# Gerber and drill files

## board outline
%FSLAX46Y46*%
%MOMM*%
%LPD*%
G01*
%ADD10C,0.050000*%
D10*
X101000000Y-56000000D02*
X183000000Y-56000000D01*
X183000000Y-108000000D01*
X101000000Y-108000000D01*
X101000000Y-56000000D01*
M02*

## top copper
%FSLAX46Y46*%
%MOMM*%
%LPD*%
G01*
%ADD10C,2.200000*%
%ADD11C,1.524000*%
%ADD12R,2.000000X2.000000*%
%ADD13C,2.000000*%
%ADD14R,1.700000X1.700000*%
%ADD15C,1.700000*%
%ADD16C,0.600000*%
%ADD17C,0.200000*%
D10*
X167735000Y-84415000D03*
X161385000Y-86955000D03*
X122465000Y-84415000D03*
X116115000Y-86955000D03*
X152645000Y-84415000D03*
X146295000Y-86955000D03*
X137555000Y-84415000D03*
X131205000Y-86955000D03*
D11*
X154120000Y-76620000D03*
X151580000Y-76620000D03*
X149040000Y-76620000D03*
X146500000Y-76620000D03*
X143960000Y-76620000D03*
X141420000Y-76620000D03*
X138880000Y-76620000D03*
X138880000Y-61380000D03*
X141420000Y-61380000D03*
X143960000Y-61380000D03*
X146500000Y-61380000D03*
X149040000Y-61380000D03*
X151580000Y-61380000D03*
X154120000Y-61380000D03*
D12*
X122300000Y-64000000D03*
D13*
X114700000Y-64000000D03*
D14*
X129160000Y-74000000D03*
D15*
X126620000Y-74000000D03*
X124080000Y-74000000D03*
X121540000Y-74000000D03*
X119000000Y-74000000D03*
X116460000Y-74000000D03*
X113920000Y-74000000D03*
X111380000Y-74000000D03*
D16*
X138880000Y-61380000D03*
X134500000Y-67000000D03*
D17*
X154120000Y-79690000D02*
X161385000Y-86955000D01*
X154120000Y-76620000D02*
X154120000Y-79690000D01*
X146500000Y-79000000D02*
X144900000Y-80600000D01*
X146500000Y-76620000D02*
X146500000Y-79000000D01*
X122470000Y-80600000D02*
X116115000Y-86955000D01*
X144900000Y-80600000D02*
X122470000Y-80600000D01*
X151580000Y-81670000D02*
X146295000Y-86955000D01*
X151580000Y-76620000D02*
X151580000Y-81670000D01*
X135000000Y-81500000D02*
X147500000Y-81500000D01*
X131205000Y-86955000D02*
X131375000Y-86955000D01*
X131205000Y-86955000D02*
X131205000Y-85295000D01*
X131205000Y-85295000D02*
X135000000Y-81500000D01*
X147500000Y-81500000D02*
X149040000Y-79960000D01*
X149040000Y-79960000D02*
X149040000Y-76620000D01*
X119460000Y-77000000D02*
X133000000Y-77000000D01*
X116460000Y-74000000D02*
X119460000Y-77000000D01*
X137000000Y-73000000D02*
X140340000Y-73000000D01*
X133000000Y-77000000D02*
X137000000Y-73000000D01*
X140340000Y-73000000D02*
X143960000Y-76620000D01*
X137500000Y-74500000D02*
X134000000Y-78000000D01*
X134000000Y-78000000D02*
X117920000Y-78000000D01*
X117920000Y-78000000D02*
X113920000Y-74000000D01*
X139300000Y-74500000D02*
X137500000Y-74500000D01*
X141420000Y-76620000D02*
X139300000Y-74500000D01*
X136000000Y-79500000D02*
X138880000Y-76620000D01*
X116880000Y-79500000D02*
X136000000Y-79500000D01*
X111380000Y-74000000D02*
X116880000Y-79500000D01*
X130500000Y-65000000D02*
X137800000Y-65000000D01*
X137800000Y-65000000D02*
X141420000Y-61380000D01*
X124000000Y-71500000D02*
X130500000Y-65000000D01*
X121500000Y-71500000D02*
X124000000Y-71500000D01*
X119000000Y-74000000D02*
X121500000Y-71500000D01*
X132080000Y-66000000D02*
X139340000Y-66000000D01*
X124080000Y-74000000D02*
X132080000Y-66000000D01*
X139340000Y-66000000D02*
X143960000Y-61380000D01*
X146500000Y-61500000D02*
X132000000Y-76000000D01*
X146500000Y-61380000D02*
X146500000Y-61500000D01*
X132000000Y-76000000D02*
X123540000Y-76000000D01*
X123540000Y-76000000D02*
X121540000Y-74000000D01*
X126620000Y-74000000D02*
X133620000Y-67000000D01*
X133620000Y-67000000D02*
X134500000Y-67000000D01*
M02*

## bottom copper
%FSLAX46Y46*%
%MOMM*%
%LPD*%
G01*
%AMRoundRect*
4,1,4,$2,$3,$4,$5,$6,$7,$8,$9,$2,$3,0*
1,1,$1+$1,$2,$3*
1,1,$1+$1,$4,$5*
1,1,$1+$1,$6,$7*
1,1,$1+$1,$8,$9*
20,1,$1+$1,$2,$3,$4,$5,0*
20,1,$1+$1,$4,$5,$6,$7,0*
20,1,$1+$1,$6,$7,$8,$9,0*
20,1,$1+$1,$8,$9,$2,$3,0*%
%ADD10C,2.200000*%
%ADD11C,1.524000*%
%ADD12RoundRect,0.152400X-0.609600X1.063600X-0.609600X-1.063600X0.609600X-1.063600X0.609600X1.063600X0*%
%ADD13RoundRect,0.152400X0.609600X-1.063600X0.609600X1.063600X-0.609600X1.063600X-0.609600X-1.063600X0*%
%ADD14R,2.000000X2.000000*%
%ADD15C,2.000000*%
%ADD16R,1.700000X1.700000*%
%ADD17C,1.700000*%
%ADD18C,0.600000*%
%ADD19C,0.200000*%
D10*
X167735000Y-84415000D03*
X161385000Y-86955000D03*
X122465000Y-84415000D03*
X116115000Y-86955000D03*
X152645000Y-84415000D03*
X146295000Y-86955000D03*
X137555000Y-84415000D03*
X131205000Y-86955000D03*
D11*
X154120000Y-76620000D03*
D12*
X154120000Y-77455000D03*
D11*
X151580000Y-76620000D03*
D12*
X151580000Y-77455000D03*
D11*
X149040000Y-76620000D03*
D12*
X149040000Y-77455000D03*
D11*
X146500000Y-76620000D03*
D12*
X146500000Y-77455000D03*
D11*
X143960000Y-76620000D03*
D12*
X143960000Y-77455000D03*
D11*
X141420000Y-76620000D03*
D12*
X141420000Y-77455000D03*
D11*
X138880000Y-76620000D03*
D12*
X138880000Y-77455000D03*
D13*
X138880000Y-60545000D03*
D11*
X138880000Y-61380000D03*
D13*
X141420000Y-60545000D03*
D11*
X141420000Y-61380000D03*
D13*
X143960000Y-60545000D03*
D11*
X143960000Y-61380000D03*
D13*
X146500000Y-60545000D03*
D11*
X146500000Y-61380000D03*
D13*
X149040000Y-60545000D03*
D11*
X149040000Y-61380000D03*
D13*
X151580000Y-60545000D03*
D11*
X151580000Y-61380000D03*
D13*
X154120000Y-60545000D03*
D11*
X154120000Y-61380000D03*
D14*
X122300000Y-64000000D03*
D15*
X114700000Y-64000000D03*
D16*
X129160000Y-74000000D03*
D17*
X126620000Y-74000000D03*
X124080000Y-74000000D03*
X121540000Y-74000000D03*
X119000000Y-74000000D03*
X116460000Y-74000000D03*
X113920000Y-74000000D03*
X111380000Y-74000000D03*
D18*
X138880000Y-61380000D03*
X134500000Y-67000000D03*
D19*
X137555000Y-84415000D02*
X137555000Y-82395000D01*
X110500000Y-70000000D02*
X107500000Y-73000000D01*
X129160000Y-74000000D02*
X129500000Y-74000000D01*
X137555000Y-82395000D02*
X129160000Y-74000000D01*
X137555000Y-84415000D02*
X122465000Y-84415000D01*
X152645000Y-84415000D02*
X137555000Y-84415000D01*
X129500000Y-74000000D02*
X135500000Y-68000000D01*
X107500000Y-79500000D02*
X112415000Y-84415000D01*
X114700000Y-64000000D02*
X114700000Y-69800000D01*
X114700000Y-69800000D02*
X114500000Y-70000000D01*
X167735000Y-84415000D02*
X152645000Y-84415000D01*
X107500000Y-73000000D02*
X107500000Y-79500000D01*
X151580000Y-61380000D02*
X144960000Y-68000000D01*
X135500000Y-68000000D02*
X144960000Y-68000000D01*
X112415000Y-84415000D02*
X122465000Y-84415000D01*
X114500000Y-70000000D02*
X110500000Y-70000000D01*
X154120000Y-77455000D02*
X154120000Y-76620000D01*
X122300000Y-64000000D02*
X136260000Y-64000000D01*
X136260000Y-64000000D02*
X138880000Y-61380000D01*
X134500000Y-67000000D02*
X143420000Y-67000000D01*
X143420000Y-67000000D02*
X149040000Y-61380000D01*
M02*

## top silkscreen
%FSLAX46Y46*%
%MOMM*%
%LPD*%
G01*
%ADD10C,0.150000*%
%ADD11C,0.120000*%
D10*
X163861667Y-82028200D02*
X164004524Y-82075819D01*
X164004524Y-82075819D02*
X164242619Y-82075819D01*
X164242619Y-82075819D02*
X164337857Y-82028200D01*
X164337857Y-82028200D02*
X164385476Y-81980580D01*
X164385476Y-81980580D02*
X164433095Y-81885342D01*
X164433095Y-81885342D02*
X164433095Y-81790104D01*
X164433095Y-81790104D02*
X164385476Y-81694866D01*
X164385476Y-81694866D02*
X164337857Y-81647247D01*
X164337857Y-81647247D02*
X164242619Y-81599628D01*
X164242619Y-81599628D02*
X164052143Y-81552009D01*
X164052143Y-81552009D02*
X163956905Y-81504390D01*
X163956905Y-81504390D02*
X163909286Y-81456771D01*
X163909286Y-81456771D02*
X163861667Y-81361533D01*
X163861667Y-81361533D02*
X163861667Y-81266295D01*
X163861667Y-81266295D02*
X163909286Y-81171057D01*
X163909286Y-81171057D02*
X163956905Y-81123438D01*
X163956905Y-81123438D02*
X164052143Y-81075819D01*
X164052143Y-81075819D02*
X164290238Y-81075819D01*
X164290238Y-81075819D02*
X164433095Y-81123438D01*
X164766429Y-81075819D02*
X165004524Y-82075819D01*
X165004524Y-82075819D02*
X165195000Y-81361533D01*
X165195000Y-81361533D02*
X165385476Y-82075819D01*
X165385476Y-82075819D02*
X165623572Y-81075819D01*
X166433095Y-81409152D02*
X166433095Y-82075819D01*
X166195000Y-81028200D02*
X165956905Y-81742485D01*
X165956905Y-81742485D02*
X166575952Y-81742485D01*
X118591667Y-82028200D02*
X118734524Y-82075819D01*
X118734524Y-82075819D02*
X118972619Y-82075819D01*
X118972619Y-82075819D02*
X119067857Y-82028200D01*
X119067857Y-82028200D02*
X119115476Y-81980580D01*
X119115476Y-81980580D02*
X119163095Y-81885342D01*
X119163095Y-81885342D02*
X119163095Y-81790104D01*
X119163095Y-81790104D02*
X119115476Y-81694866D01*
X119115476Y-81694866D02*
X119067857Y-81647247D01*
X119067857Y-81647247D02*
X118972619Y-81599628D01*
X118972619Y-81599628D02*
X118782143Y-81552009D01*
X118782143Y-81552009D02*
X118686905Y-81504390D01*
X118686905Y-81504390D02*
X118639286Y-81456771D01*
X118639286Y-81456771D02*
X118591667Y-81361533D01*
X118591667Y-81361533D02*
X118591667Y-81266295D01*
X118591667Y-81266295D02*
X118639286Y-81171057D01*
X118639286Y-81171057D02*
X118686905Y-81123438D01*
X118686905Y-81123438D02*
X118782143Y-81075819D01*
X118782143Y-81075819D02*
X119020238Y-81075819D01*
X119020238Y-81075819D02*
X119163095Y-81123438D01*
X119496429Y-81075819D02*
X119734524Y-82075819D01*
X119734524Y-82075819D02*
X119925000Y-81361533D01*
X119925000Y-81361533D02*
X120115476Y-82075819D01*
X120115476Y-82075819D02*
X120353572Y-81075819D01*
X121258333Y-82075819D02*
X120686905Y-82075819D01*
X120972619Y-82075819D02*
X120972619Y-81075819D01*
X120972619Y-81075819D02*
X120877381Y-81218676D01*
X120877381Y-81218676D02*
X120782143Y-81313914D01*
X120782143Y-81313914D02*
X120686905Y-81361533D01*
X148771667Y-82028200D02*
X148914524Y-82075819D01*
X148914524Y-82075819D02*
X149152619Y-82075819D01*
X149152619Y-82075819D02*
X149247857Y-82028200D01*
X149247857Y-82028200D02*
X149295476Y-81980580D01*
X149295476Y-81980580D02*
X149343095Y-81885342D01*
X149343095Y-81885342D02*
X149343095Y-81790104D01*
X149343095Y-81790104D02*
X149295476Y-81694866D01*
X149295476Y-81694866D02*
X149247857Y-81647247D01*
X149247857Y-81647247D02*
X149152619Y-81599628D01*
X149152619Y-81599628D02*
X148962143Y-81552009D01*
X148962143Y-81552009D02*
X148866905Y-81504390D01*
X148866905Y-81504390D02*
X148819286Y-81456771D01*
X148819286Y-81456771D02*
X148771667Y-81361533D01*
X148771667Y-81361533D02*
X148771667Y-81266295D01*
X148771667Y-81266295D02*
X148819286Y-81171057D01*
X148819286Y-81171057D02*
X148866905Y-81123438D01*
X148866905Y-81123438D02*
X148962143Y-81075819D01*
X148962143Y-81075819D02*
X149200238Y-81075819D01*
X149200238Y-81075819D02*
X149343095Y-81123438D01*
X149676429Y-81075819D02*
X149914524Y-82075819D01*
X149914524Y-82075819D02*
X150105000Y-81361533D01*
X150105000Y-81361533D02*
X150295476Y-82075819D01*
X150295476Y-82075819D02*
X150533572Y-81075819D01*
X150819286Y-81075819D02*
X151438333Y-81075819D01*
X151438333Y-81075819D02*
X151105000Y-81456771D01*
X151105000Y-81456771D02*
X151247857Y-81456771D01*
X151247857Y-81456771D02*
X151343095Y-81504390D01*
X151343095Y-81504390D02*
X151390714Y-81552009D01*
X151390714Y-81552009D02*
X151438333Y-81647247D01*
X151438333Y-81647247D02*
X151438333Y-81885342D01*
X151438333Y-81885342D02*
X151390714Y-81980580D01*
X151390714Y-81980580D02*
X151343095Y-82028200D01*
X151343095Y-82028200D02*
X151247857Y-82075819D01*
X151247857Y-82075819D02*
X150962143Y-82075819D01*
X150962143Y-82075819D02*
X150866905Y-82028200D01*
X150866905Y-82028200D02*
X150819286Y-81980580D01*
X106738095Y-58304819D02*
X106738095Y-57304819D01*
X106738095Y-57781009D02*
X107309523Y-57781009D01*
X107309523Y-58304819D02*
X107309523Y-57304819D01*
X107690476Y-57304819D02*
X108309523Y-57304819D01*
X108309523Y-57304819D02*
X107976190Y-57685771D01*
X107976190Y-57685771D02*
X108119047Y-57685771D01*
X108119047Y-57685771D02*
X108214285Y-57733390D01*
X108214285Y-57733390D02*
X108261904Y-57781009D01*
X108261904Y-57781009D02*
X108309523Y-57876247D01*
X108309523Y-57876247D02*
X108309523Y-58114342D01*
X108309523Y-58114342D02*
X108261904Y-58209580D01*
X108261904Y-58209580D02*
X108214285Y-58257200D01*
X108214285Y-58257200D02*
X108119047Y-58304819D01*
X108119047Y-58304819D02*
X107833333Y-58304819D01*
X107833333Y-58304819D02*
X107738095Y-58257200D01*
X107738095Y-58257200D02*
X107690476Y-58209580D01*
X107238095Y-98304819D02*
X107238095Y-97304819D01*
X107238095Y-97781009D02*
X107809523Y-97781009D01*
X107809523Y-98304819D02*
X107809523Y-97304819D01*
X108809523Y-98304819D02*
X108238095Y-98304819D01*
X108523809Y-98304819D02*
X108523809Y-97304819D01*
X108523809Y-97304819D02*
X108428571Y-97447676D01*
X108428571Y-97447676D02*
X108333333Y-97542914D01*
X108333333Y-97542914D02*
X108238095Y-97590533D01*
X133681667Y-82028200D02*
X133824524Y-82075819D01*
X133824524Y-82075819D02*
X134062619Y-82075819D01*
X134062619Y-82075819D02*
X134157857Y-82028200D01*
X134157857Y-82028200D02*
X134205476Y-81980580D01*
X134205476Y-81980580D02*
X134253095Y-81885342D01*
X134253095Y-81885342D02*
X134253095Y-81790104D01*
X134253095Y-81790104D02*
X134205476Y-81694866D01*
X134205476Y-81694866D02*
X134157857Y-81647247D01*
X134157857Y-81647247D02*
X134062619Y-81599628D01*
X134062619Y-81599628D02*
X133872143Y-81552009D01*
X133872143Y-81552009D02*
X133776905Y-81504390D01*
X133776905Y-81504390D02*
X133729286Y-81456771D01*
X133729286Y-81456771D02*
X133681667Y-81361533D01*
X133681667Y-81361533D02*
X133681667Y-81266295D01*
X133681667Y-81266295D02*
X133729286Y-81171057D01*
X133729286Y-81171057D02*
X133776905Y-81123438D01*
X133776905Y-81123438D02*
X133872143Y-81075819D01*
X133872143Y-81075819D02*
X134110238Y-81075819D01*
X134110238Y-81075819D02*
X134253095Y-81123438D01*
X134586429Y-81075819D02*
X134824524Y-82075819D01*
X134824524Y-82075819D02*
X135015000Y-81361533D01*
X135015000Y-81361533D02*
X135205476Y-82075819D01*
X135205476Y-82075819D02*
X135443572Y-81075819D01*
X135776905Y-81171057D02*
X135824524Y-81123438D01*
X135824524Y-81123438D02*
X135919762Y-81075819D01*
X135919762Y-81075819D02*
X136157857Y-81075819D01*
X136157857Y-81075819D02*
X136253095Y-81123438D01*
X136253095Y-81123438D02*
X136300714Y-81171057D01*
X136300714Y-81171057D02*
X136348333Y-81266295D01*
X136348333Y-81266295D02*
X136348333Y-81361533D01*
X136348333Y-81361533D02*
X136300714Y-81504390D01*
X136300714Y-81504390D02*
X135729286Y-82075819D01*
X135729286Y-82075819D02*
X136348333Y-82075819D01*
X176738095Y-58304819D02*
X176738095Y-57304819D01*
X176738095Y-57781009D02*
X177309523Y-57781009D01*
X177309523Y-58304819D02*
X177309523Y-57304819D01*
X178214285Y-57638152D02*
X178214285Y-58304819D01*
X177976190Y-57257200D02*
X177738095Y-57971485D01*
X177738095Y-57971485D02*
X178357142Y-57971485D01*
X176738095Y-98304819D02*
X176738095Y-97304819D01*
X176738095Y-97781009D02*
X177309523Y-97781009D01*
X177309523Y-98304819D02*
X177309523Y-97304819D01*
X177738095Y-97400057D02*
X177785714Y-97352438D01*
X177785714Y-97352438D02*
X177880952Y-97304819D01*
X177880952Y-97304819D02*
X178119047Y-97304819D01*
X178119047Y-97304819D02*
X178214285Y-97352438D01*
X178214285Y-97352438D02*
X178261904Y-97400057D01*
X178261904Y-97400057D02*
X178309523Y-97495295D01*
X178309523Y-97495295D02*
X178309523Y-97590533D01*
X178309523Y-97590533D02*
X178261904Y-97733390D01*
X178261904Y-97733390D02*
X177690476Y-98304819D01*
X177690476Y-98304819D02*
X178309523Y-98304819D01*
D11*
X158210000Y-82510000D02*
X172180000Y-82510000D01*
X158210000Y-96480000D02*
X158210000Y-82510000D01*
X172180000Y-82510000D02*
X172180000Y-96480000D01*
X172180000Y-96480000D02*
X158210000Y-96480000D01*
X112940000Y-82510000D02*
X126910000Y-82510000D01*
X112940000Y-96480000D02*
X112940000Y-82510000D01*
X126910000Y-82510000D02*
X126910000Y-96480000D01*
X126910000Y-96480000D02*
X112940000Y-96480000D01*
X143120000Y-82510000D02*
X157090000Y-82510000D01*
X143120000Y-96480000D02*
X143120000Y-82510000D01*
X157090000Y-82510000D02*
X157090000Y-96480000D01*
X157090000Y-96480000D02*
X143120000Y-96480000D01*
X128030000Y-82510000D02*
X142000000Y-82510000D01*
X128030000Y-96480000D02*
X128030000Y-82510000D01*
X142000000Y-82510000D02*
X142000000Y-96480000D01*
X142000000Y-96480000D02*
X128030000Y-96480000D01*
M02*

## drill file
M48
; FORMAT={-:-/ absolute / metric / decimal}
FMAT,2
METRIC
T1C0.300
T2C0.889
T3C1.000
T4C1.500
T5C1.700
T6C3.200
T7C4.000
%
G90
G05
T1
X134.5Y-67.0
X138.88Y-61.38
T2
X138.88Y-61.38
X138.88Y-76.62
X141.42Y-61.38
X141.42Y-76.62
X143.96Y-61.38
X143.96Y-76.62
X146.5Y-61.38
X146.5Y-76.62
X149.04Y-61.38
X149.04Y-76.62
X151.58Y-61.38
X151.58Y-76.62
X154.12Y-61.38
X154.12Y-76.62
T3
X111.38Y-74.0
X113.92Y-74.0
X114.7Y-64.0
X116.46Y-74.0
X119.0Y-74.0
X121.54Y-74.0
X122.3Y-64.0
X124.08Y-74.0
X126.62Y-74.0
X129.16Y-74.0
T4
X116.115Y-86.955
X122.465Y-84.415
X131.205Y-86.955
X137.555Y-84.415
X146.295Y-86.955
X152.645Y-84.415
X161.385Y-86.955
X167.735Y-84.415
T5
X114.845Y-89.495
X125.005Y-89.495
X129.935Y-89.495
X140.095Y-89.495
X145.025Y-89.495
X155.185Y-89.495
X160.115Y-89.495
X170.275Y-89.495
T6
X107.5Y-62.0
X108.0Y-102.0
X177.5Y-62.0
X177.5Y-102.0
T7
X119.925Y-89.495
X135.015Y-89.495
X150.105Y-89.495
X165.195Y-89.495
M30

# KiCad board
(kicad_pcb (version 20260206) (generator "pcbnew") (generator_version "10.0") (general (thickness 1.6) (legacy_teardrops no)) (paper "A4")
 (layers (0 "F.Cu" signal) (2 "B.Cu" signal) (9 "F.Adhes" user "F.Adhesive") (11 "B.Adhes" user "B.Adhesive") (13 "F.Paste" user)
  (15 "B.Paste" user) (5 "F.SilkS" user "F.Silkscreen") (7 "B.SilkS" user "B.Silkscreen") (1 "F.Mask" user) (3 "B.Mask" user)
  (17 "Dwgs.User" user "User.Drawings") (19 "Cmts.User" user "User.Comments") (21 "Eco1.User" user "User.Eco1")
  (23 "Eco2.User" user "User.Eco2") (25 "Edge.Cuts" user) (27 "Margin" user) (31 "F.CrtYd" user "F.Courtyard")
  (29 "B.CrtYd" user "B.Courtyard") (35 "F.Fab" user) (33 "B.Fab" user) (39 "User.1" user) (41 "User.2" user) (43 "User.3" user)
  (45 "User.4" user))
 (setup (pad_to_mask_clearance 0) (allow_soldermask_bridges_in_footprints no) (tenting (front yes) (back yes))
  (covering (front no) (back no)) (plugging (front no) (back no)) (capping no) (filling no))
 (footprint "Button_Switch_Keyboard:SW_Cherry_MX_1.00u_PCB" (layer "F.Cu") (at 167.735 84.415)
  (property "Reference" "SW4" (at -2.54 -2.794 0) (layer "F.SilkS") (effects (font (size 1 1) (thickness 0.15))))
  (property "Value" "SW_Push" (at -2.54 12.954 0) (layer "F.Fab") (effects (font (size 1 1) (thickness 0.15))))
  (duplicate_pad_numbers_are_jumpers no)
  (fp_line (start -9.525 -1.905) (end 4.445 -1.905) (stroke (width 0.12) (type solid)) (layer "F.SilkS"))
  (fp_line (start -9.525 12.065) (end -9.525 -1.905) (stroke (width 0.12) (type solid)) (layer "F.SilkS"))
  (fp_line (start 4.445 -1.905) (end 4.445 12.065) (stroke (width 0.12) (type solid)) (layer "F.SilkS"))
  (fp_line (start 4.445 12.065) (end -9.525 12.065) (stroke (width 0.12) (type solid)) (layer "F.SilkS"))
  (pad "" np_thru_hole circle (at -7.62 5.08) (size 1.7 1.7) (drill 1.7) (layers "*.Cu" "*.Mask"))
  (pad "" np_thru_hole circle (at -2.54 5.08) (size 4 4) (drill 4) (layers "*.Cu" "*.Mask"))
  (pad "" np_thru_hole circle (at 2.54 5.08) (size 1.7 1.7) (drill 1.7) (layers "*.Cu" "*.Mask"))
  (pad "1" thru_hole circle (at 0 0) (size 2.2 2.2) (drill 1.5) (layers "*.Cu" "*.Mask") (remove_unused_layers no) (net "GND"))
  (pad "2" thru_hole circle (at -6.35 2.54) (size 2.2 2.2) (drill 1.5) (layers "*.Cu" "*.Mask") (remove_unused_layers no)
   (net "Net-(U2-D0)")))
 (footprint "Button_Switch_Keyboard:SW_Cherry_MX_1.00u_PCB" (layer "F.Cu") (at 122.465 84.415)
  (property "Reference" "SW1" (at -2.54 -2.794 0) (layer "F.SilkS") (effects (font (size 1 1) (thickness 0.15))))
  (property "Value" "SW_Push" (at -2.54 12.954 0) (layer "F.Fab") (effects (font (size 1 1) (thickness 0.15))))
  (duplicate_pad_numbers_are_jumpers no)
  (fp_line (start -9.525 -1.905) (end 4.445 -1.905) (stroke (width 0.12) (type solid)) (layer "F.SilkS"))
  (fp_line (start -9.525 12.065) (end -9.525 -1.905) (stroke (width 0.12) (type solid)) (layer "F.SilkS"))
  (fp_line (start 4.445 -1.905) (end 4.445 12.065) (stroke (width 0.12) (type solid)) (layer "F.SilkS"))
  (fp_line (start 4.445 12.065) (end -9.525 12.065) (stroke (width 0.12) (type solid)) (layer "F.SilkS"))
  (pad "" np_thru_hole circle (at -7.62 5.08) (size 1.7 1.7) (drill 1.7) (layers "*.Cu" "*.Mask"))
  (pad "" np_thru_hole circle (at -2.54 5.08) (size 4 4) (drill 4) (layers "*.Cu" "*.Mask"))
  (pad "" np_thru_hole circle (at 2.54 5.08) (size 1.7 1.7) (drill 1.7) (layers "*.Cu" "*.Mask"))
  (pad "1" thru_hole circle (at 0 0) (size 2.2 2.2) (drill 1.5) (layers "*.Cu" "*.Mask") (remove_unused_layers no) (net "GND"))
  (pad "2" thru_hole circle (at -6.35 2.54) (size 2.2 2.2) (drill 1.5) (layers "*.Cu" "*.Mask") (remove_unused_layers no)
   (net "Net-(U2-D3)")))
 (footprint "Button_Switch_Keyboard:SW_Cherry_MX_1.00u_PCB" (layer "F.Cu") (at 152.645 84.415)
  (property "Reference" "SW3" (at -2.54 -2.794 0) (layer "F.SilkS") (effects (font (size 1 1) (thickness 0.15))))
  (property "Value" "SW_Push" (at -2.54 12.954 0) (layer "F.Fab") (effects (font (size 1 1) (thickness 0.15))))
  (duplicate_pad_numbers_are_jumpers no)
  (fp_line (start -9.525 -1.905) (end 4.445 -1.905) (stroke (width 0.12) (type solid)) (layer "F.SilkS"))
  (fp_line (start -9.525 12.065) (end -9.525 -1.905) (stroke (width 0.12) (type solid)) (layer "F.SilkS"))
  (fp_line (start 4.445 -1.905) (end 4.445 12.065) (stroke (width 0.12) (type solid)) (layer "F.SilkS"))
  (fp_line (start 4.445 12.065) (end -9.525 12.065) (stroke (width 0.12) (type solid)) (layer "F.SilkS"))
  (pad "" np_thru_hole circle (at -7.62 5.08) (size 1.7 1.7) (drill 1.7) (layers "*.Cu" "*.Mask"))
  (pad "" np_thru_hole circle (at -2.54 5.08) (size 4 4) (drill 4) (layers "*.Cu" "*.Mask"))
  (pad "" np_thru_hole circle (at 2.54 5.08) (size 1.7 1.7) (drill 1.7) (layers "*.Cu" "*.Mask"))
  (pad "1" thru_hole circle (at 0 0) (size 2.2 2.2) (drill 1.5) (layers "*.Cu" "*.Mask") (remove_unused_layers no) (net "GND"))
  (pad "2" thru_hole circle (at -6.35 2.54) (size 2.2 2.2) (drill 1.5) (layers "*.Cu" "*.Mask") (remove_unused_layers no)
   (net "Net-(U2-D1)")))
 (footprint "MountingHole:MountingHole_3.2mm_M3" (layer "F.Cu") (at 107.5 62)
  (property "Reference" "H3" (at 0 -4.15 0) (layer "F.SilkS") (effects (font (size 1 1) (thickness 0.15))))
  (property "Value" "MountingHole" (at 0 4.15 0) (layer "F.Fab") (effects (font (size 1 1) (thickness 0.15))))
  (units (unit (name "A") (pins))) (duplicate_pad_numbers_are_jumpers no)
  (pad "" np_thru_hole circle (at 0 0) (size 3.2 3.2) (drill 3.2) (layers "*.Cu" "*.Mask")))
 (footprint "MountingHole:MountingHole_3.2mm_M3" (layer "F.Cu") (at 108 102)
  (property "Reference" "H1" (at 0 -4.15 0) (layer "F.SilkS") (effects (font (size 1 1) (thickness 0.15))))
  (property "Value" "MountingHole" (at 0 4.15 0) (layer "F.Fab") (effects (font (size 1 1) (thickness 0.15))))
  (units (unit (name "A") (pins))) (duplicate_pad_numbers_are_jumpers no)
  (pad "" np_thru_hole circle (at 0 0) (size 3.2 3.2) (drill 3.2) (layers "*.Cu" "*.Mask")))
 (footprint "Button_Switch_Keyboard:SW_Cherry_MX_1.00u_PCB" (layer "F.Cu") (at 137.555 84.415)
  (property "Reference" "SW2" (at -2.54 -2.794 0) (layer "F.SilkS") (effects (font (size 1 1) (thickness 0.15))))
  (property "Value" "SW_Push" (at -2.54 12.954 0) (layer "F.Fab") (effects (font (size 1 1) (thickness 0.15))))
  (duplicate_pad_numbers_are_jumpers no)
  (fp_line (start -9.525 -1.905) (end 4.445 -1.905) (stroke (width 0.12) (type solid)) (layer "F.SilkS"))
  (fp_line (start -9.525 12.065) (end -9.525 -1.905) (stroke (width 0.12) (type solid)) (layer "F.SilkS"))
  (fp_line (start 4.445 -1.905) (end 4.445 12.065) (stroke (width 0.12) (type solid)) (layer "F.SilkS"))
  (fp_line (start 4.445 12.065) (end -9.525 12.065) (stroke (width 0.12) (type solid)) (layer "F.SilkS"))
  (pad "" np_thru_hole circle (at -7.62 5.08) (size 1.7 1.7) (drill 1.7) (layers "*.Cu" "*.Mask"))
  (pad "" np_thru_hole circle (at -2.54 5.08) (size 4 4) (drill 4) (layers "*.Cu" "*.Mask"))
  (pad "" np_thru_hole circle (at 2.54 5.08) (size 1.7 1.7) (drill 1.7) (layers "*.Cu" "*.Mask"))
  (pad "1" thru_hole circle (at 0 0) (size 2.2 2.2) (drill 1.5) (layers "*.Cu" "*.Mask") (remove_unused_layers no) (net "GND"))
  (pad "2" thru_hole circle (at -6.35 2.54) (size 2.2 2.2) (drill 1.5) (layers "*.Cu" "*.Mask") (remove_unused_layers no)
   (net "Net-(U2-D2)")))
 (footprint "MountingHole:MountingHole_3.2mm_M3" (layer "F.Cu") (at 177.5 62)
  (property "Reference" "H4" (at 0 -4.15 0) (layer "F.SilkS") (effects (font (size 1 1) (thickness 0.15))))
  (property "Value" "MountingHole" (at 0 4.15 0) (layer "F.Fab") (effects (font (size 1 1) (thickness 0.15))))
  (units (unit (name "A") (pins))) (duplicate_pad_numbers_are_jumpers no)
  (pad "" np_thru_hole circle (at 0 0) (size 3.2 3.2) (drill 3.2) (layers "*.Cu" "*.Mask")))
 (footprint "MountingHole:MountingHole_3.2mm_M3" (layer "F.Cu") (at 177.5 102)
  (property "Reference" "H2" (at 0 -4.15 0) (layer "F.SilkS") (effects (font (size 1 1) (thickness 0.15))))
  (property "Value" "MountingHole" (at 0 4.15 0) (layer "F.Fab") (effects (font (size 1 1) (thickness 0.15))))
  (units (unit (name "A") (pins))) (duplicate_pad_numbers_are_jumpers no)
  (pad "" np_thru_hole circle (at 0 0) (size 3.2 3.2) (drill 3.2) (layers "*.Cu" "*.Mask")))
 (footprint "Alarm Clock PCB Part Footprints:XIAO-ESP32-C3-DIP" (layer "B.Cu") (at 146.5 69)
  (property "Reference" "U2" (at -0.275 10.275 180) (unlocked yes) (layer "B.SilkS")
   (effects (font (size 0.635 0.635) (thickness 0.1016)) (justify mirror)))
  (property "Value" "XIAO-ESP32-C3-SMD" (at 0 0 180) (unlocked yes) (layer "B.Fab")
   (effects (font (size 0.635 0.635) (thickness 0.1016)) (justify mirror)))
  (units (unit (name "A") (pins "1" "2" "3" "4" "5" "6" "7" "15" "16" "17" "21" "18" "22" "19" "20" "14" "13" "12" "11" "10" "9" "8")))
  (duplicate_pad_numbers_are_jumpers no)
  (pad "1" thru_hole circle (at 7.62 7.62 270) (size 1.524 1.524) (drill 0.889) (layers "*.Cu" "*.Mask") (remove_unused_layers no)
   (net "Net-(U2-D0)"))
  (pad "1" smd roundrect (at 7.62 8.455 270) (size 2.432 1.524) (layers "B.Cu" "B.Mask") (roundrect_rratio 0.1) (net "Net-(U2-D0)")
   (thermal_bridge_angle 45))
  (pad "2" thru_hole circle (at 5.08 7.62 270) (size 1.524 1.524) (drill 0.889) (layers "*.Cu" "*.Mask") (remove_unused_layers no)
   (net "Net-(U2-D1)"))
  (pad "2" smd roundrect (at 5.08 8.455 270) (size 2.432 1.524) (layers "B.Cu" "B.Mask") (roundrect_rratio 0.1) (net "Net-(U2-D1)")
   (thermal_bridge_angle 45))
  (pad "3" thru_hole circle (at 2.54 7.62 270) (size 1.524 1.524) (drill 0.889) (layers "*.Cu" "*.Mask") (remove_unused_layers no)
   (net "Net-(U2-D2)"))
  (pad "3" smd roundrect (at 2.54 8.455 270) (size 2.432 1.524) (layers "B.Cu" "B.Mask") (roundrect_rratio 0.1) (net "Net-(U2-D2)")
   (thermal_bridge_angle 45))
  (pad "4" thru_hole circle (at 0 7.62 270) (size 1.524 1.524) (drill 0.889) (layers "*.Cu" "*.Mask") (remove_unused_layers no)
   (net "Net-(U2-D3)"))
  (pad "4" smd roundrect (at 0 8.455 270) (size 2.432 1.524) (layers "B.Cu" "B.Mask") (roundrect_rratio 0.1) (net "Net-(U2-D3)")
   (thermal_bridge_angle 45))
  (pad "5" thru_hole circle (at -2.54 7.62 270) (size 1.524 1.524) (drill 0.889) (layers "*.Cu" "*.Mask") (remove_unused_layers no)
   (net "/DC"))
  (pad "5" smd roundrect (at -2.54 8.455 270) (size 2.432 1.524) (layers "B.Cu" "B.Mask") (roundrect_rratio 0.1) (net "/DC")
   (thermal_bridge_angle 45))
  (pad "6" thru_hole circle (at -5.08 7.62 270) (size 1.524 1.524) (drill 0.889) (layers "*.Cu" "*.Mask") (remove_unused_layers no)
   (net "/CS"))
  (pad "6" smd roundrect (at -5.08 8.455 270) (size 2.432 1.524) (layers "B.Cu" "B.Mask") (roundrect_rratio 0.1) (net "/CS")
   (thermal_bridge_angle 45))
  (pad "7" thru_hole circle (at -7.62 7.62 270) (size 1.524 1.524) (drill 0.889) (layers "*.Cu" "*.Mask") (remove_unused_layers no)
   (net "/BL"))
  (pad "7" smd roundrect (at -7.62 8.455 270) (size 2.432 1.524) (layers "B.Cu" "B.Mask") (roundrect_rratio 0.1) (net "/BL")
   (thermal_bridge_angle 45))
  (pad "8" smd roundrect (at -7.62 -8.455 90) (size 2.432 1.524) (layers "B.Cu" "B.Mask") (roundrect_rratio 0.1) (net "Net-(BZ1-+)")
   (thermal_bridge_angle 45))
  (pad "8" thru_hole circle (at -7.62 -7.62 90) (size 1.524 1.524) (drill 0.889) (layers "*.Cu" "*.Mask") (remove_unused_layers no)
   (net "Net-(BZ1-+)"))
  (pad "9" smd roundrect (at -5.08 -8.455 90) (size 2.432 1.524) (layers "B.Cu" "B.Mask") (roundrect_rratio 0.1) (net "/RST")
   (thermal_bridge_angle 45))
  (pad "9" thru_hole circle (at -5.08 -7.62 90) (size 1.524 1.524) (drill 0.889) (layers "*.Cu" "*.Mask") (remove_unused_layers no)
   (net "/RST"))
  (pad "10" smd roundrect (at -2.54 -8.455 90) (size 2.432 1.524) (layers "B.Cu" "B.Mask") (roundrect_rratio 0.1) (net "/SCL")
   (thermal_bridge_angle 45))
  (pad "10" thru_hole circle (at -2.54 -7.62 90) (size 1.524 1.524) (drill 0.889) (layers "*.Cu" "*.Mask") (remove_unused_layers no)
   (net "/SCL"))
  (pad "11" smd roundrect (at 0 -8.455 90) (size 2.432 1.524) (layers "B.Cu" "B.Mask") (roundrect_rratio 0.1) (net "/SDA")
   (thermal_bridge_angle 45))
  (pad "11" thru_hole circle (at 0 -7.62 90) (size 1.524 1.524) (drill 0.889) (layers "*.Cu" "*.Mask") (remove_unused_layers no)
   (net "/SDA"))
  (pad "12" smd roundrect (at 2.54 -8.455 90) (size 2.432 1.524) (layers "B.Cu" "B.Mask") (roundrect_rratio 0.1) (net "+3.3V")
   (thermal_bridge_angle 45))
  (pad "12" thru_hole circle (at 2.54 -7.62 90) (size 1.524 1.524) (drill 0.889) (layers "*.Cu" "*.Mask") (remove_unused_layers no)
   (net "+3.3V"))
  (pad "13" smd roundrect (at 5.08 -8.455 90) (size 2.432 1.524) (layers "B.Cu" "B.Mask") (roundrect_rratio 0.1) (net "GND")
   (thermal_bridge_angle 45))
  (pad "13" thru_hole circle (at 5.08 -7.62 90) (size 1.524 1.524) (drill 0.889) (layers "*.Cu" "*.Mask") (remove_unused_layers no)
   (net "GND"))
  (pad "14" smd roundrect (at 7.62 -8.455 90) (size 2.432 1.524) (layers "B.Cu" "B.Mask") (roundrect_rratio 0.1)
   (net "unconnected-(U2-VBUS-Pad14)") (thermal_bridge_angle 45))
  (pad "14" thru_hole circle (at 7.62 -7.62 90) (size 1.524 1.524) (drill 0.889) (layers "*.Cu" "*.Mask") (remove_unused_layers no)
   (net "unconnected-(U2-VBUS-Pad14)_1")))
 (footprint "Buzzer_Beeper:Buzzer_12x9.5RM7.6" (layer "B.Cu") (at 122.3 64 180)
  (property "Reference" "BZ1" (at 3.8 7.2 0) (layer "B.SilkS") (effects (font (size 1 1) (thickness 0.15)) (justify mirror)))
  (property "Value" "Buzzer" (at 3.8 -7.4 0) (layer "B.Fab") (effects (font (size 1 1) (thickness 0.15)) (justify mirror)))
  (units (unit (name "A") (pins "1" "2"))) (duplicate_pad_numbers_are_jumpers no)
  (pad "1" thru_hole rect (at 0 0 180) (size 2 2) (drill 1) (layers "*.Cu" "*.Mask") (remove_unused_layers no) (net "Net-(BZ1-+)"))
  (pad "2" thru_hole circle (at 7.6 0 180) (size 2 2) (drill 1) (layers "*.Cu" "*.Mask") (remove_unused_layers no) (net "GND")))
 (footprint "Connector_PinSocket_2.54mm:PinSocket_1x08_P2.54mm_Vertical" (layer "B.Cu") (at 129.16 74 90)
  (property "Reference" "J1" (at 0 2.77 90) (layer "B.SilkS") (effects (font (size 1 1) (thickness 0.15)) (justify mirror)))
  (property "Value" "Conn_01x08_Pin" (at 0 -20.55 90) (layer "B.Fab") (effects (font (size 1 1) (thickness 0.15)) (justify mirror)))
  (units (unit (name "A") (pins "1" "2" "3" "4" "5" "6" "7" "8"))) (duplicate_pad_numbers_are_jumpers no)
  (pad "1" thru_hole rect (at 0 0 90) (size 1.7 1.7) (drill 1) (layers "*.Cu" "*.Mask") (remove_unused_layers no) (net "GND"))
  (pad "2" thru_hole circle (at 0 -2.54 90) (size 1.7 1.7) (drill 1) (layers "*.Cu" "*.Mask") (remove_unused_layers no) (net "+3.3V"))
  (pad "3" thru_hole circle (at 0 -5.08 90) (size 1.7 1.7) (drill 1) (layers "*.Cu" "*.Mask") (remove_unused_layers no) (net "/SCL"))
  (pad "4" thru_hole circle (at 0 -7.62 90) (size 1.7 1.7) (drill 1) (layers "*.Cu" "*.Mask") (remove_unused_layers no) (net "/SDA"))
  (pad "5" thru_hole circle (at 0 -10.16 90) (size 1.7 1.7) (drill 1) (layers "*.Cu" "*.Mask") (remove_unused_layers no) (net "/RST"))
  (pad "6" thru_hole circle (at 0 -12.7 90) (size 1.7 1.7) (drill 1) (layers "*.Cu" "*.Mask") (remove_unused_layers no) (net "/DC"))
  (pad "7" thru_hole circle (at 0 -15.24 90) (size 1.7 1.7) (drill 1) (layers "*.Cu" "*.Mask") (remove_unused_layers no) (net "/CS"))
  (pad "8" thru_hole circle (at 0 -17.78 90) (size 1.7 1.7) (drill 1) (layers "*.Cu" "*.Mask") (remove_unused_layers no) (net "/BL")))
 (gr_rect (start 101 56) (end 183 108) (stroke (width 0.05) (type default)) (fill no) (layer "Edge.Cuts"))
 (segment (start 137.555 84.415) (end 137.555 82.395) (width 0.2) (layer "B.Cu") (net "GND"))
 (segment (start 110.5 70) (end 107.5 73) (width 0.2) (layer "B.Cu") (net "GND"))
 (segment (start 129.16 74) (end 129.5 74) (width 0.2) (layer "B.Cu") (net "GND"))
 (segment (start 137.555 82.395) (end 129.16 74) (width 0.2) (layer "B.Cu") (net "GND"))
 (segment (start 137.555 84.415) (end 122.465 84.415) (width 0.2) (layer "B.Cu") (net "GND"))
 (segment (start 152.645 84.415) (end 137.555 84.415) (width 0.2) (layer "B.Cu") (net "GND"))
 (segment (start 129.5 74) (end 135.5 68) (width 0.2) (layer "B.Cu") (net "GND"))
 (segment (start 107.5 79.5) (end 112.415 84.415) (width 0.2) (layer "B.Cu") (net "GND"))
 (segment (start 114.7 64) (end 114.7 69.8) (width 0.2) (layer "B.Cu") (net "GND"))
 (segment (start 114.7 69.8) (end 114.5 70) (width 0.2) (layer "B.Cu") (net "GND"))
 (segment (start 167.735 84.415) (end 152.645 84.415) (width 0.2) (layer "B.Cu") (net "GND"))
 (segment (start 107.5 73) (end 107.5 79.5) (width 0.2) (layer "B.Cu") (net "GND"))
 (segment (start 151.58 61.38) (end 144.96 68) (width 0.2) (layer "B.Cu") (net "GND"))
 (segment (start 135.5 68) (end 144.96 68) (width 0.2) (layer "B.Cu") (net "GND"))
 (segment (start 112.415 84.415) (end 122.465 84.415) (width 0.2) (layer "B.Cu") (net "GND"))
 (segment (start 114.5 70) (end 110.5 70) (width 0.2) (layer "B.Cu") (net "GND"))
 (segment (start 154.12 79.69) (end 161.385 86.955) (width 0.2) (layer "F.Cu") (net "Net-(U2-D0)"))
 (segment (start 154.12 76.62) (end 154.12 79.69) (width 0.2) (layer "F.Cu") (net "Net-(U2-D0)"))
 (segment (start 154.12 77.455) (end 154.12 76.62) (width 0.2) (layer "B.Cu") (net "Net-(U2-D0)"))
 (segment (start 146.5 79) (end 144.9 80.6) (width 0.2) (layer "F.Cu") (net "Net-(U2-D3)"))
 (segment (start 146.5 76.62) (end 146.5 79) (width 0.2) (layer "F.Cu") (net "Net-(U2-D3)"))
 (segment (start 122.47 80.6) (end 116.115 86.955) (width 0.2) (layer "F.Cu") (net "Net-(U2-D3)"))
 (segment (start 144.9 80.6) (end 122.47 80.6) (width 0.2) (layer "F.Cu") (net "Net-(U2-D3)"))
 (segment (start 151.58 81.67) (end 146.295 86.955) (width 0.2) (layer "F.Cu") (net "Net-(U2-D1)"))
 (segment (start 151.58 76.62) (end 151.58 81.67) (width 0.2) (layer "F.Cu") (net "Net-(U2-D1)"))
 (segment (start 135 81.5) (end 147.5 81.5) (width 0.2) (layer "F.Cu") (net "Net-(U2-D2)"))
 (segment (start 131.205 86.955) (end 131.375 86.955) (width 0.2) (layer "F.Cu") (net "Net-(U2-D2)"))
 (segment (start 131.205 86.955) (end 131.205 85.295) (width 0.2) (layer "F.Cu") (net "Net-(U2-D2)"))
 (segment (start 131.205 85.295) (end 135 81.5) (width 0.2) (layer "F.Cu") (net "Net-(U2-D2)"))
 (segment (start 147.5 81.5) (end 149.04 79.96) (width 0.2) (layer "F.Cu") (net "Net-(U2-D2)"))
 (segment (start 149.04 79.96) (end 149.04 76.62) (width 0.2) (layer "F.Cu") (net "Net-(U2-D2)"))
 (segment (start 119.46 77) (end 133 77) (width 0.2) (layer "F.Cu") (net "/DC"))
 (segment (start 116.46 74) (end 119.46 77) (width 0.2) (layer "F.Cu") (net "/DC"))
 (segment (start 137 73) (end 140.34 73) (width 0.2) (layer "F.Cu") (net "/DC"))
 (segment (start 133 77) (end 137 73) (width 0.2) (layer "F.Cu") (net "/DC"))
 (segment (start 140.34 73) (end 143.96 76.62) (width 0.2) (layer "F.Cu") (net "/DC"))
 (segment (start 137.5 74.5) (end 134 78) (width 0.2) (layer "F.Cu") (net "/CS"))
 (segment (start 134 78) (end 117.92 78) (width 0.2) (layer "F.Cu") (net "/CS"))
 (segment (start 117.92 78) (end 113.92 74) (width 0.2) (layer "F.Cu") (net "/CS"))
 (segment (start 139.3 74.5) (end 137.5 74.5) (width 0.2) (layer "F.Cu") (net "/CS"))
 (segment (start 141.42 76.62) (end 139.3 74.5) (width 0.2) (layer "F.Cu") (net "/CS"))
 (segment (start 136 79.5) (end 138.88 76.62) (width 0.2) (layer "F.Cu") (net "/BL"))
 (segment (start 116.88 79.5) (end 136 79.5) (width 0.2) (layer "F.Cu") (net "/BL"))
 (segment (start 111.38 74) (end 116.88 79.5) (width 0.2) (layer "F.Cu") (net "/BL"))
 (via (at 138.88 61.38) (size 0.6) (drill 0.3) (layers "F.Cu" "B.Cu") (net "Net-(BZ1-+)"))
 (segment (start 122.3 64) (end 136.26 64) (width 0.2) (layer "B.Cu") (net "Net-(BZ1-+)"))
 (segment (start 136.26 64) (end 138.88 61.38) (width 0.2) (layer "B.Cu") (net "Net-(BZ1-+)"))
 (segment (start 130.5 65) (end 137.8 65) (width 0.2) (layer "F.Cu") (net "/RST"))
 (segment (start 137.8 65) (end 141.42 61.38) (width 0.2) (layer "F.Cu") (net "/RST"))
 (segment (start 124 71.5) (end 130.5 65) (width 0.2) (layer "F.Cu") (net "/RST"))
 (segment (start 121.5 71.5) (end 124 71.5) (width 0.2) (layer "F.Cu") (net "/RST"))
 (segment (start 119 74) (end 121.5 71.5) (width 0.2) (layer "F.Cu") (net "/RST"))
 (segment (start 132.08 66) (end 139.34 66) (width 0.2) (layer "F.Cu") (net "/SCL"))
 (segment (start 124.08 74) (end 132.08 66) (width 0.2) (layer "F.Cu") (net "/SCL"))
 (segment (start 139.34 66) (end 143.96 61.38) (width 0.2) (layer "F.Cu") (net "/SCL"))
 (segment (start 146.5 61.5) (end 132 76) (width 0.2) (layer "F.Cu") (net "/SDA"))
 (segment (start 146.5 61.38) (end 146.5 61.5) (width 0.2) (layer "F.Cu") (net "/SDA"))
 (segment (start 132 76) (end 123.54 76) (width 0.2) (layer "F.Cu") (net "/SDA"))
 (segment (start 123.54 76) (end 121.54 74) (width 0.2) (layer "F.Cu") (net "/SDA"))
 (segment (start 126.62 74) (end 133.62 67) (width 0.2) (layer "F.Cu") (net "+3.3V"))
 (segment (start 133.62 67) (end 134.5 67) (width 0.2) (layer "F.Cu") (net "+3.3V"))
 (via (at 134.5 67) (size 0.6) (drill 0.3) (layers "F.Cu" "B.Cu") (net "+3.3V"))
 (segment (start 134.5 67) (end 143.42 67) (width 0.2) (layer "B.Cu") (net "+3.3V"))
 (segment (start 143.42 67) (end 149.04 61.38) (width 0.2) (layer "B.Cu") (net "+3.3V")))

